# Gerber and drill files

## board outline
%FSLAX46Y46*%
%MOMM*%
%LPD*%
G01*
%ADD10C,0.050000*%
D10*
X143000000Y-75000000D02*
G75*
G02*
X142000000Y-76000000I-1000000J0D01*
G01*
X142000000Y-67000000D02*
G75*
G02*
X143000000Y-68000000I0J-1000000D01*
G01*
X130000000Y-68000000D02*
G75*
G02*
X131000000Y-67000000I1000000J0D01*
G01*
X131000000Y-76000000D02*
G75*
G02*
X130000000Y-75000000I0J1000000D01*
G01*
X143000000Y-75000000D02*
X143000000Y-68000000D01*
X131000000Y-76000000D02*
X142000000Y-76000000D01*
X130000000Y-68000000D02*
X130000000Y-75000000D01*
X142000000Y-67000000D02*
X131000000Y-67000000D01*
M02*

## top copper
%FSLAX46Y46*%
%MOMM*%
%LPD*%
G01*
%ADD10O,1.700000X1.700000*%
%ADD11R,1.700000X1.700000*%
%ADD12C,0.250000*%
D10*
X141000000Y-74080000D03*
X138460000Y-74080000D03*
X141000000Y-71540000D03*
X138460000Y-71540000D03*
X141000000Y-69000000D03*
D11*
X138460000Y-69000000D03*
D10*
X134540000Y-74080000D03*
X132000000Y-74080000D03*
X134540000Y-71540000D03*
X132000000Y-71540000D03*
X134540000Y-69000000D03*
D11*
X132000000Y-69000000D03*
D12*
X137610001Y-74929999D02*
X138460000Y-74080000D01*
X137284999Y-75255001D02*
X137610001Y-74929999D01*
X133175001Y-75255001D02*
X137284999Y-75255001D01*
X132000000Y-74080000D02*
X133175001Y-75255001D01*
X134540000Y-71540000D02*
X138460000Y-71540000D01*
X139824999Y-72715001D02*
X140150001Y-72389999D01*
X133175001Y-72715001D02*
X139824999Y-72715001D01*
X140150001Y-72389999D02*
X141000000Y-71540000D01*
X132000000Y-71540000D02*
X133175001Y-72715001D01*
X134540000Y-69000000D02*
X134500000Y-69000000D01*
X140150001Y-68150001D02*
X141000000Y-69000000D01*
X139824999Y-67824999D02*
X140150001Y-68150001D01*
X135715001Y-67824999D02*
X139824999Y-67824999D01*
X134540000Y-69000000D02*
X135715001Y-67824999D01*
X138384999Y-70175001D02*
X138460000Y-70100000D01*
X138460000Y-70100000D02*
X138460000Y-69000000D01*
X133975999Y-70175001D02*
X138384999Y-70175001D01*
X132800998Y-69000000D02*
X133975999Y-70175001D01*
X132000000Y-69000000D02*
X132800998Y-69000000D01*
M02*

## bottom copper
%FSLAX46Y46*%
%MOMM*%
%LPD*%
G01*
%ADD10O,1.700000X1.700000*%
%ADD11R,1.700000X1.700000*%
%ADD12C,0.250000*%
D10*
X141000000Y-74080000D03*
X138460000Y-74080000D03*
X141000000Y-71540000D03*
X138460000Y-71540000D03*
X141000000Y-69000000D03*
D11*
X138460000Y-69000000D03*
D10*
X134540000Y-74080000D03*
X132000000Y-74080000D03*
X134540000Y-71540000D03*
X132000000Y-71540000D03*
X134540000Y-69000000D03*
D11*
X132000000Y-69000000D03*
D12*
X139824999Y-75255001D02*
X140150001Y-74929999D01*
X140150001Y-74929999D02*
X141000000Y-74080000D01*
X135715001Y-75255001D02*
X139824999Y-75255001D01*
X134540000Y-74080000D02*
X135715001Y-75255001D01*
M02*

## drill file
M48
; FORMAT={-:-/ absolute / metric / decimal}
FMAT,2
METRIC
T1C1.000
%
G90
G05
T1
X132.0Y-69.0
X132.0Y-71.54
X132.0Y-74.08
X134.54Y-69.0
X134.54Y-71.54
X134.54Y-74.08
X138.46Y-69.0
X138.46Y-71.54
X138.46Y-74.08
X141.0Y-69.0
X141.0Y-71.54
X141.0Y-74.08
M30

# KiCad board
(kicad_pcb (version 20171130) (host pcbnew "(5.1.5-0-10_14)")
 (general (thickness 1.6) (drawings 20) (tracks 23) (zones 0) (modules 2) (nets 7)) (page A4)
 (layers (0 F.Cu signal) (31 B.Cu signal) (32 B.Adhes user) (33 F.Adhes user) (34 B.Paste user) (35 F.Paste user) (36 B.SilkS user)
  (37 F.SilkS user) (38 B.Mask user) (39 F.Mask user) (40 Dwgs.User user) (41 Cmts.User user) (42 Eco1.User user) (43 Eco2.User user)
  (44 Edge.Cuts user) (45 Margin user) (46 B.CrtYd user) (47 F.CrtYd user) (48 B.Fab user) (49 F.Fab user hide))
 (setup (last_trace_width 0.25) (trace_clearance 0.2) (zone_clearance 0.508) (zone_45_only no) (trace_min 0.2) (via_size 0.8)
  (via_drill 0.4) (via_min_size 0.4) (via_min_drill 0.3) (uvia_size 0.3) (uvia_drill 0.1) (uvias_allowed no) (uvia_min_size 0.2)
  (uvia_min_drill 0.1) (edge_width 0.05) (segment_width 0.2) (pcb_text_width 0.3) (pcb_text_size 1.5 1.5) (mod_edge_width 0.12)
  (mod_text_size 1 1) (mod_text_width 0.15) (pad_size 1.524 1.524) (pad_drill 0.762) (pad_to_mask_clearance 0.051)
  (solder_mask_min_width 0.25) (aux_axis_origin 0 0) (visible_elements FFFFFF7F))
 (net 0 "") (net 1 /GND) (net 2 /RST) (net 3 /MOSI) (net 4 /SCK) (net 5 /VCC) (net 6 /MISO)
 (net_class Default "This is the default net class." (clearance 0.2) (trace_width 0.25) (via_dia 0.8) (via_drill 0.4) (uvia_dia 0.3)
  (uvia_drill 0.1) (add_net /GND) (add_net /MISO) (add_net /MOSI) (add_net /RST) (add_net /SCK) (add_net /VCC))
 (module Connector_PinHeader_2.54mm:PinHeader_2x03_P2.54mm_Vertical (layer F.Cu) (at 138.46 69)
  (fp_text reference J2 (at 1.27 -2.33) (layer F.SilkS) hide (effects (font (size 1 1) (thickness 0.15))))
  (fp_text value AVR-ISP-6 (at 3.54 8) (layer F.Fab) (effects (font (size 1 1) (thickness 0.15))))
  (pad 6 thru_hole oval (at 2.54 5.08) (size 1.7 1.7) (drill 1) (layers *.Cu *.Mask) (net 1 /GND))
  (pad 5 thru_hole oval (at 0 5.08) (size 1.7 1.7) (drill 1) (layers *.Cu *.Mask) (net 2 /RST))
  (pad 4 thru_hole oval (at 2.54 2.54) (size 1.7 1.7) (drill 1) (layers *.Cu *.Mask) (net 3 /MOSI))
  (pad 3 thru_hole oval (at 0 2.54) (size 1.7 1.7) (drill 1) (layers *.Cu *.Mask) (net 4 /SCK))
  (pad 2 thru_hole oval (at 2.54 0) (size 1.7 1.7) (drill 1) (layers *.Cu *.Mask) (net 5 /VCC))
  (pad 1 thru_hole rect (at 0 0) (size 1.7 1.7) (drill 1) (layers *.Cu *.Mask) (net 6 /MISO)))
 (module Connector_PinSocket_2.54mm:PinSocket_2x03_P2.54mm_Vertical (layer B.Cu) (at 132 69 180)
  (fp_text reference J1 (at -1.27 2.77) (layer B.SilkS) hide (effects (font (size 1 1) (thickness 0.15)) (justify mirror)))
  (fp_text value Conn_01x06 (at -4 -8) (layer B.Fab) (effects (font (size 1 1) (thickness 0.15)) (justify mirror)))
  (pad 6 thru_hole oval (at -2.54 -5.08 180) (size 1.7 1.7) (drill 1) (layers *.Cu *.Mask) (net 1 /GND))
  (pad 5 thru_hole oval (at 0 -5.08 180) (size 1.7 1.7) (drill 1) (layers *.Cu *.Mask) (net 2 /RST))
  (pad 4 thru_hole oval (at -2.54 -2.54 180) (size 1.7 1.7) (drill 1) (layers *.Cu *.Mask) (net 4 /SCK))
  (pad 3 thru_hole oval (at 0 -2.54 180) (size 1.7 1.7) (drill 1) (layers *.Cu *.Mask) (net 3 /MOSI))
  (pad 2 thru_hole oval (at -2.54 0 180) (size 1.7 1.7) (drill 1) (layers *.Cu *.Mask) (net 5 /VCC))
  (pad 1 thru_hole rect (at 0 0 180) (size 1.7 1.7) (drill 1) (layers *.Cu *.Mask) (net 6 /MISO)))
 (gr_arc (start 142 75) (end 142 76) (angle -90) (layer Edge.Cuts) (width 0.05))
 (gr_arc (start 142 68) (end 143 68) (angle -90) (layer Edge.Cuts) (width 0.05))
 (gr_arc (start 131 68) (end 131 67) (angle -90) (layer Edge.Cuts) (width 0.05))
 (gr_arc (start 131 75) (end 130 75) (angle -90) (layer Edge.Cuts) (width 0.05))
 (gr_line (start 143 75) (end 143 68) (layer Edge.Cuts) (width 0.05))
 (gr_line (start 131 76) (end 142 76) (layer Edge.Cuts) (width 0.05))
 (gr_line (start 130 68) (end 130 75) (layer Edge.Cuts) (width 0.05))
 (gr_line (start 142 67) (end 131 67) (layer Edge.Cuts) (width 0.05))
 (segment (start 139.824999 75.255001) (end 140.150001 74.929999) (width 0.25) (layer B.Cu) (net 1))
 (segment (start 140.150001 74.929999) (end 141 74.08) (width 0.25) (layer B.Cu) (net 1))
 (segment (start 135.715001 75.255001) (end 139.824999 75.255001) (width 0.25) (layer B.Cu) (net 1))
 (segment (start 134.54 74.08) (end 135.715001 75.255001) (width 0.25) (layer B.Cu) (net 1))
 (segment (start 137.610001 74.929999) (end 138.46 74.08) (width 0.25) (layer F.Cu) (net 2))
 (segment (start 137.284999 75.255001) (end 137.610001 74.929999) (width 0.25) (layer F.Cu) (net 2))
 (segment (start 133.175001 75.255001) (end 137.284999 75.255001) (width 0.25) (layer F.Cu) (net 2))
 (segment (start 132 74.08) (end 133.175001 75.255001) (width 0.25) (layer F.Cu) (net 2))
 (segment (start 134.54 71.54) (end 138.46 71.54) (width 0.25) (layer F.Cu) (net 4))
 (segment (start 139.824999 72.715001) (end 140.150001 72.389999) (width 0.25) (layer F.Cu) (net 3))
 (segment (start 133.175001 72.715001) (end 139.824999 72.715001) (width 0.25) (layer F.Cu) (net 3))
 (segment (start 140.150001 72.389999) (end 141 71.54) (width 0.25) (layer F.Cu) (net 3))
 (segment (start 132 71.54) (end 133.175001 72.715001) (width 0.25) (layer F.Cu) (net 3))
 (segment (start 134.54 69) (end 134.5 69) (width 0.25) (layer F.Cu) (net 5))
 (segment (start 140.150001 68.150001) (end 141 69) (width 0.25) (layer F.Cu) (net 5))
 (segment (start 139.824999 67.824999) (end 140.150001 68.150001) (width 0.25) (layer F.Cu) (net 5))
 (segment (start 135.715001 67.824999) (end 139.824999 67.824999) (width 0.25) (layer F.Cu) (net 5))
 (segment (start 134.54 69) (end 135.715001 67.824999) (width 0.25) (layer F.Cu) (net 5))
 (segment (start 138.384999 70.175001) (end 138.46 70.1) (width 0.25) (layer F.Cu) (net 6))
 (segment (start 138.46 70.1) (end 138.46 69) (width 0.25) (layer F.Cu) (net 6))
 (segment (start 133.975999 70.175001) (end 138.384999 70.175001) (width 0.25) (layer F.Cu) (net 6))
 (segment (start 132.800998 69) (end 133.975999 70.175001) (width 0.25) (layer F.Cu) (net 6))
 (segment (start 132 69) (end 132.800998 69) (width 0.25) (layer F.Cu) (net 6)))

